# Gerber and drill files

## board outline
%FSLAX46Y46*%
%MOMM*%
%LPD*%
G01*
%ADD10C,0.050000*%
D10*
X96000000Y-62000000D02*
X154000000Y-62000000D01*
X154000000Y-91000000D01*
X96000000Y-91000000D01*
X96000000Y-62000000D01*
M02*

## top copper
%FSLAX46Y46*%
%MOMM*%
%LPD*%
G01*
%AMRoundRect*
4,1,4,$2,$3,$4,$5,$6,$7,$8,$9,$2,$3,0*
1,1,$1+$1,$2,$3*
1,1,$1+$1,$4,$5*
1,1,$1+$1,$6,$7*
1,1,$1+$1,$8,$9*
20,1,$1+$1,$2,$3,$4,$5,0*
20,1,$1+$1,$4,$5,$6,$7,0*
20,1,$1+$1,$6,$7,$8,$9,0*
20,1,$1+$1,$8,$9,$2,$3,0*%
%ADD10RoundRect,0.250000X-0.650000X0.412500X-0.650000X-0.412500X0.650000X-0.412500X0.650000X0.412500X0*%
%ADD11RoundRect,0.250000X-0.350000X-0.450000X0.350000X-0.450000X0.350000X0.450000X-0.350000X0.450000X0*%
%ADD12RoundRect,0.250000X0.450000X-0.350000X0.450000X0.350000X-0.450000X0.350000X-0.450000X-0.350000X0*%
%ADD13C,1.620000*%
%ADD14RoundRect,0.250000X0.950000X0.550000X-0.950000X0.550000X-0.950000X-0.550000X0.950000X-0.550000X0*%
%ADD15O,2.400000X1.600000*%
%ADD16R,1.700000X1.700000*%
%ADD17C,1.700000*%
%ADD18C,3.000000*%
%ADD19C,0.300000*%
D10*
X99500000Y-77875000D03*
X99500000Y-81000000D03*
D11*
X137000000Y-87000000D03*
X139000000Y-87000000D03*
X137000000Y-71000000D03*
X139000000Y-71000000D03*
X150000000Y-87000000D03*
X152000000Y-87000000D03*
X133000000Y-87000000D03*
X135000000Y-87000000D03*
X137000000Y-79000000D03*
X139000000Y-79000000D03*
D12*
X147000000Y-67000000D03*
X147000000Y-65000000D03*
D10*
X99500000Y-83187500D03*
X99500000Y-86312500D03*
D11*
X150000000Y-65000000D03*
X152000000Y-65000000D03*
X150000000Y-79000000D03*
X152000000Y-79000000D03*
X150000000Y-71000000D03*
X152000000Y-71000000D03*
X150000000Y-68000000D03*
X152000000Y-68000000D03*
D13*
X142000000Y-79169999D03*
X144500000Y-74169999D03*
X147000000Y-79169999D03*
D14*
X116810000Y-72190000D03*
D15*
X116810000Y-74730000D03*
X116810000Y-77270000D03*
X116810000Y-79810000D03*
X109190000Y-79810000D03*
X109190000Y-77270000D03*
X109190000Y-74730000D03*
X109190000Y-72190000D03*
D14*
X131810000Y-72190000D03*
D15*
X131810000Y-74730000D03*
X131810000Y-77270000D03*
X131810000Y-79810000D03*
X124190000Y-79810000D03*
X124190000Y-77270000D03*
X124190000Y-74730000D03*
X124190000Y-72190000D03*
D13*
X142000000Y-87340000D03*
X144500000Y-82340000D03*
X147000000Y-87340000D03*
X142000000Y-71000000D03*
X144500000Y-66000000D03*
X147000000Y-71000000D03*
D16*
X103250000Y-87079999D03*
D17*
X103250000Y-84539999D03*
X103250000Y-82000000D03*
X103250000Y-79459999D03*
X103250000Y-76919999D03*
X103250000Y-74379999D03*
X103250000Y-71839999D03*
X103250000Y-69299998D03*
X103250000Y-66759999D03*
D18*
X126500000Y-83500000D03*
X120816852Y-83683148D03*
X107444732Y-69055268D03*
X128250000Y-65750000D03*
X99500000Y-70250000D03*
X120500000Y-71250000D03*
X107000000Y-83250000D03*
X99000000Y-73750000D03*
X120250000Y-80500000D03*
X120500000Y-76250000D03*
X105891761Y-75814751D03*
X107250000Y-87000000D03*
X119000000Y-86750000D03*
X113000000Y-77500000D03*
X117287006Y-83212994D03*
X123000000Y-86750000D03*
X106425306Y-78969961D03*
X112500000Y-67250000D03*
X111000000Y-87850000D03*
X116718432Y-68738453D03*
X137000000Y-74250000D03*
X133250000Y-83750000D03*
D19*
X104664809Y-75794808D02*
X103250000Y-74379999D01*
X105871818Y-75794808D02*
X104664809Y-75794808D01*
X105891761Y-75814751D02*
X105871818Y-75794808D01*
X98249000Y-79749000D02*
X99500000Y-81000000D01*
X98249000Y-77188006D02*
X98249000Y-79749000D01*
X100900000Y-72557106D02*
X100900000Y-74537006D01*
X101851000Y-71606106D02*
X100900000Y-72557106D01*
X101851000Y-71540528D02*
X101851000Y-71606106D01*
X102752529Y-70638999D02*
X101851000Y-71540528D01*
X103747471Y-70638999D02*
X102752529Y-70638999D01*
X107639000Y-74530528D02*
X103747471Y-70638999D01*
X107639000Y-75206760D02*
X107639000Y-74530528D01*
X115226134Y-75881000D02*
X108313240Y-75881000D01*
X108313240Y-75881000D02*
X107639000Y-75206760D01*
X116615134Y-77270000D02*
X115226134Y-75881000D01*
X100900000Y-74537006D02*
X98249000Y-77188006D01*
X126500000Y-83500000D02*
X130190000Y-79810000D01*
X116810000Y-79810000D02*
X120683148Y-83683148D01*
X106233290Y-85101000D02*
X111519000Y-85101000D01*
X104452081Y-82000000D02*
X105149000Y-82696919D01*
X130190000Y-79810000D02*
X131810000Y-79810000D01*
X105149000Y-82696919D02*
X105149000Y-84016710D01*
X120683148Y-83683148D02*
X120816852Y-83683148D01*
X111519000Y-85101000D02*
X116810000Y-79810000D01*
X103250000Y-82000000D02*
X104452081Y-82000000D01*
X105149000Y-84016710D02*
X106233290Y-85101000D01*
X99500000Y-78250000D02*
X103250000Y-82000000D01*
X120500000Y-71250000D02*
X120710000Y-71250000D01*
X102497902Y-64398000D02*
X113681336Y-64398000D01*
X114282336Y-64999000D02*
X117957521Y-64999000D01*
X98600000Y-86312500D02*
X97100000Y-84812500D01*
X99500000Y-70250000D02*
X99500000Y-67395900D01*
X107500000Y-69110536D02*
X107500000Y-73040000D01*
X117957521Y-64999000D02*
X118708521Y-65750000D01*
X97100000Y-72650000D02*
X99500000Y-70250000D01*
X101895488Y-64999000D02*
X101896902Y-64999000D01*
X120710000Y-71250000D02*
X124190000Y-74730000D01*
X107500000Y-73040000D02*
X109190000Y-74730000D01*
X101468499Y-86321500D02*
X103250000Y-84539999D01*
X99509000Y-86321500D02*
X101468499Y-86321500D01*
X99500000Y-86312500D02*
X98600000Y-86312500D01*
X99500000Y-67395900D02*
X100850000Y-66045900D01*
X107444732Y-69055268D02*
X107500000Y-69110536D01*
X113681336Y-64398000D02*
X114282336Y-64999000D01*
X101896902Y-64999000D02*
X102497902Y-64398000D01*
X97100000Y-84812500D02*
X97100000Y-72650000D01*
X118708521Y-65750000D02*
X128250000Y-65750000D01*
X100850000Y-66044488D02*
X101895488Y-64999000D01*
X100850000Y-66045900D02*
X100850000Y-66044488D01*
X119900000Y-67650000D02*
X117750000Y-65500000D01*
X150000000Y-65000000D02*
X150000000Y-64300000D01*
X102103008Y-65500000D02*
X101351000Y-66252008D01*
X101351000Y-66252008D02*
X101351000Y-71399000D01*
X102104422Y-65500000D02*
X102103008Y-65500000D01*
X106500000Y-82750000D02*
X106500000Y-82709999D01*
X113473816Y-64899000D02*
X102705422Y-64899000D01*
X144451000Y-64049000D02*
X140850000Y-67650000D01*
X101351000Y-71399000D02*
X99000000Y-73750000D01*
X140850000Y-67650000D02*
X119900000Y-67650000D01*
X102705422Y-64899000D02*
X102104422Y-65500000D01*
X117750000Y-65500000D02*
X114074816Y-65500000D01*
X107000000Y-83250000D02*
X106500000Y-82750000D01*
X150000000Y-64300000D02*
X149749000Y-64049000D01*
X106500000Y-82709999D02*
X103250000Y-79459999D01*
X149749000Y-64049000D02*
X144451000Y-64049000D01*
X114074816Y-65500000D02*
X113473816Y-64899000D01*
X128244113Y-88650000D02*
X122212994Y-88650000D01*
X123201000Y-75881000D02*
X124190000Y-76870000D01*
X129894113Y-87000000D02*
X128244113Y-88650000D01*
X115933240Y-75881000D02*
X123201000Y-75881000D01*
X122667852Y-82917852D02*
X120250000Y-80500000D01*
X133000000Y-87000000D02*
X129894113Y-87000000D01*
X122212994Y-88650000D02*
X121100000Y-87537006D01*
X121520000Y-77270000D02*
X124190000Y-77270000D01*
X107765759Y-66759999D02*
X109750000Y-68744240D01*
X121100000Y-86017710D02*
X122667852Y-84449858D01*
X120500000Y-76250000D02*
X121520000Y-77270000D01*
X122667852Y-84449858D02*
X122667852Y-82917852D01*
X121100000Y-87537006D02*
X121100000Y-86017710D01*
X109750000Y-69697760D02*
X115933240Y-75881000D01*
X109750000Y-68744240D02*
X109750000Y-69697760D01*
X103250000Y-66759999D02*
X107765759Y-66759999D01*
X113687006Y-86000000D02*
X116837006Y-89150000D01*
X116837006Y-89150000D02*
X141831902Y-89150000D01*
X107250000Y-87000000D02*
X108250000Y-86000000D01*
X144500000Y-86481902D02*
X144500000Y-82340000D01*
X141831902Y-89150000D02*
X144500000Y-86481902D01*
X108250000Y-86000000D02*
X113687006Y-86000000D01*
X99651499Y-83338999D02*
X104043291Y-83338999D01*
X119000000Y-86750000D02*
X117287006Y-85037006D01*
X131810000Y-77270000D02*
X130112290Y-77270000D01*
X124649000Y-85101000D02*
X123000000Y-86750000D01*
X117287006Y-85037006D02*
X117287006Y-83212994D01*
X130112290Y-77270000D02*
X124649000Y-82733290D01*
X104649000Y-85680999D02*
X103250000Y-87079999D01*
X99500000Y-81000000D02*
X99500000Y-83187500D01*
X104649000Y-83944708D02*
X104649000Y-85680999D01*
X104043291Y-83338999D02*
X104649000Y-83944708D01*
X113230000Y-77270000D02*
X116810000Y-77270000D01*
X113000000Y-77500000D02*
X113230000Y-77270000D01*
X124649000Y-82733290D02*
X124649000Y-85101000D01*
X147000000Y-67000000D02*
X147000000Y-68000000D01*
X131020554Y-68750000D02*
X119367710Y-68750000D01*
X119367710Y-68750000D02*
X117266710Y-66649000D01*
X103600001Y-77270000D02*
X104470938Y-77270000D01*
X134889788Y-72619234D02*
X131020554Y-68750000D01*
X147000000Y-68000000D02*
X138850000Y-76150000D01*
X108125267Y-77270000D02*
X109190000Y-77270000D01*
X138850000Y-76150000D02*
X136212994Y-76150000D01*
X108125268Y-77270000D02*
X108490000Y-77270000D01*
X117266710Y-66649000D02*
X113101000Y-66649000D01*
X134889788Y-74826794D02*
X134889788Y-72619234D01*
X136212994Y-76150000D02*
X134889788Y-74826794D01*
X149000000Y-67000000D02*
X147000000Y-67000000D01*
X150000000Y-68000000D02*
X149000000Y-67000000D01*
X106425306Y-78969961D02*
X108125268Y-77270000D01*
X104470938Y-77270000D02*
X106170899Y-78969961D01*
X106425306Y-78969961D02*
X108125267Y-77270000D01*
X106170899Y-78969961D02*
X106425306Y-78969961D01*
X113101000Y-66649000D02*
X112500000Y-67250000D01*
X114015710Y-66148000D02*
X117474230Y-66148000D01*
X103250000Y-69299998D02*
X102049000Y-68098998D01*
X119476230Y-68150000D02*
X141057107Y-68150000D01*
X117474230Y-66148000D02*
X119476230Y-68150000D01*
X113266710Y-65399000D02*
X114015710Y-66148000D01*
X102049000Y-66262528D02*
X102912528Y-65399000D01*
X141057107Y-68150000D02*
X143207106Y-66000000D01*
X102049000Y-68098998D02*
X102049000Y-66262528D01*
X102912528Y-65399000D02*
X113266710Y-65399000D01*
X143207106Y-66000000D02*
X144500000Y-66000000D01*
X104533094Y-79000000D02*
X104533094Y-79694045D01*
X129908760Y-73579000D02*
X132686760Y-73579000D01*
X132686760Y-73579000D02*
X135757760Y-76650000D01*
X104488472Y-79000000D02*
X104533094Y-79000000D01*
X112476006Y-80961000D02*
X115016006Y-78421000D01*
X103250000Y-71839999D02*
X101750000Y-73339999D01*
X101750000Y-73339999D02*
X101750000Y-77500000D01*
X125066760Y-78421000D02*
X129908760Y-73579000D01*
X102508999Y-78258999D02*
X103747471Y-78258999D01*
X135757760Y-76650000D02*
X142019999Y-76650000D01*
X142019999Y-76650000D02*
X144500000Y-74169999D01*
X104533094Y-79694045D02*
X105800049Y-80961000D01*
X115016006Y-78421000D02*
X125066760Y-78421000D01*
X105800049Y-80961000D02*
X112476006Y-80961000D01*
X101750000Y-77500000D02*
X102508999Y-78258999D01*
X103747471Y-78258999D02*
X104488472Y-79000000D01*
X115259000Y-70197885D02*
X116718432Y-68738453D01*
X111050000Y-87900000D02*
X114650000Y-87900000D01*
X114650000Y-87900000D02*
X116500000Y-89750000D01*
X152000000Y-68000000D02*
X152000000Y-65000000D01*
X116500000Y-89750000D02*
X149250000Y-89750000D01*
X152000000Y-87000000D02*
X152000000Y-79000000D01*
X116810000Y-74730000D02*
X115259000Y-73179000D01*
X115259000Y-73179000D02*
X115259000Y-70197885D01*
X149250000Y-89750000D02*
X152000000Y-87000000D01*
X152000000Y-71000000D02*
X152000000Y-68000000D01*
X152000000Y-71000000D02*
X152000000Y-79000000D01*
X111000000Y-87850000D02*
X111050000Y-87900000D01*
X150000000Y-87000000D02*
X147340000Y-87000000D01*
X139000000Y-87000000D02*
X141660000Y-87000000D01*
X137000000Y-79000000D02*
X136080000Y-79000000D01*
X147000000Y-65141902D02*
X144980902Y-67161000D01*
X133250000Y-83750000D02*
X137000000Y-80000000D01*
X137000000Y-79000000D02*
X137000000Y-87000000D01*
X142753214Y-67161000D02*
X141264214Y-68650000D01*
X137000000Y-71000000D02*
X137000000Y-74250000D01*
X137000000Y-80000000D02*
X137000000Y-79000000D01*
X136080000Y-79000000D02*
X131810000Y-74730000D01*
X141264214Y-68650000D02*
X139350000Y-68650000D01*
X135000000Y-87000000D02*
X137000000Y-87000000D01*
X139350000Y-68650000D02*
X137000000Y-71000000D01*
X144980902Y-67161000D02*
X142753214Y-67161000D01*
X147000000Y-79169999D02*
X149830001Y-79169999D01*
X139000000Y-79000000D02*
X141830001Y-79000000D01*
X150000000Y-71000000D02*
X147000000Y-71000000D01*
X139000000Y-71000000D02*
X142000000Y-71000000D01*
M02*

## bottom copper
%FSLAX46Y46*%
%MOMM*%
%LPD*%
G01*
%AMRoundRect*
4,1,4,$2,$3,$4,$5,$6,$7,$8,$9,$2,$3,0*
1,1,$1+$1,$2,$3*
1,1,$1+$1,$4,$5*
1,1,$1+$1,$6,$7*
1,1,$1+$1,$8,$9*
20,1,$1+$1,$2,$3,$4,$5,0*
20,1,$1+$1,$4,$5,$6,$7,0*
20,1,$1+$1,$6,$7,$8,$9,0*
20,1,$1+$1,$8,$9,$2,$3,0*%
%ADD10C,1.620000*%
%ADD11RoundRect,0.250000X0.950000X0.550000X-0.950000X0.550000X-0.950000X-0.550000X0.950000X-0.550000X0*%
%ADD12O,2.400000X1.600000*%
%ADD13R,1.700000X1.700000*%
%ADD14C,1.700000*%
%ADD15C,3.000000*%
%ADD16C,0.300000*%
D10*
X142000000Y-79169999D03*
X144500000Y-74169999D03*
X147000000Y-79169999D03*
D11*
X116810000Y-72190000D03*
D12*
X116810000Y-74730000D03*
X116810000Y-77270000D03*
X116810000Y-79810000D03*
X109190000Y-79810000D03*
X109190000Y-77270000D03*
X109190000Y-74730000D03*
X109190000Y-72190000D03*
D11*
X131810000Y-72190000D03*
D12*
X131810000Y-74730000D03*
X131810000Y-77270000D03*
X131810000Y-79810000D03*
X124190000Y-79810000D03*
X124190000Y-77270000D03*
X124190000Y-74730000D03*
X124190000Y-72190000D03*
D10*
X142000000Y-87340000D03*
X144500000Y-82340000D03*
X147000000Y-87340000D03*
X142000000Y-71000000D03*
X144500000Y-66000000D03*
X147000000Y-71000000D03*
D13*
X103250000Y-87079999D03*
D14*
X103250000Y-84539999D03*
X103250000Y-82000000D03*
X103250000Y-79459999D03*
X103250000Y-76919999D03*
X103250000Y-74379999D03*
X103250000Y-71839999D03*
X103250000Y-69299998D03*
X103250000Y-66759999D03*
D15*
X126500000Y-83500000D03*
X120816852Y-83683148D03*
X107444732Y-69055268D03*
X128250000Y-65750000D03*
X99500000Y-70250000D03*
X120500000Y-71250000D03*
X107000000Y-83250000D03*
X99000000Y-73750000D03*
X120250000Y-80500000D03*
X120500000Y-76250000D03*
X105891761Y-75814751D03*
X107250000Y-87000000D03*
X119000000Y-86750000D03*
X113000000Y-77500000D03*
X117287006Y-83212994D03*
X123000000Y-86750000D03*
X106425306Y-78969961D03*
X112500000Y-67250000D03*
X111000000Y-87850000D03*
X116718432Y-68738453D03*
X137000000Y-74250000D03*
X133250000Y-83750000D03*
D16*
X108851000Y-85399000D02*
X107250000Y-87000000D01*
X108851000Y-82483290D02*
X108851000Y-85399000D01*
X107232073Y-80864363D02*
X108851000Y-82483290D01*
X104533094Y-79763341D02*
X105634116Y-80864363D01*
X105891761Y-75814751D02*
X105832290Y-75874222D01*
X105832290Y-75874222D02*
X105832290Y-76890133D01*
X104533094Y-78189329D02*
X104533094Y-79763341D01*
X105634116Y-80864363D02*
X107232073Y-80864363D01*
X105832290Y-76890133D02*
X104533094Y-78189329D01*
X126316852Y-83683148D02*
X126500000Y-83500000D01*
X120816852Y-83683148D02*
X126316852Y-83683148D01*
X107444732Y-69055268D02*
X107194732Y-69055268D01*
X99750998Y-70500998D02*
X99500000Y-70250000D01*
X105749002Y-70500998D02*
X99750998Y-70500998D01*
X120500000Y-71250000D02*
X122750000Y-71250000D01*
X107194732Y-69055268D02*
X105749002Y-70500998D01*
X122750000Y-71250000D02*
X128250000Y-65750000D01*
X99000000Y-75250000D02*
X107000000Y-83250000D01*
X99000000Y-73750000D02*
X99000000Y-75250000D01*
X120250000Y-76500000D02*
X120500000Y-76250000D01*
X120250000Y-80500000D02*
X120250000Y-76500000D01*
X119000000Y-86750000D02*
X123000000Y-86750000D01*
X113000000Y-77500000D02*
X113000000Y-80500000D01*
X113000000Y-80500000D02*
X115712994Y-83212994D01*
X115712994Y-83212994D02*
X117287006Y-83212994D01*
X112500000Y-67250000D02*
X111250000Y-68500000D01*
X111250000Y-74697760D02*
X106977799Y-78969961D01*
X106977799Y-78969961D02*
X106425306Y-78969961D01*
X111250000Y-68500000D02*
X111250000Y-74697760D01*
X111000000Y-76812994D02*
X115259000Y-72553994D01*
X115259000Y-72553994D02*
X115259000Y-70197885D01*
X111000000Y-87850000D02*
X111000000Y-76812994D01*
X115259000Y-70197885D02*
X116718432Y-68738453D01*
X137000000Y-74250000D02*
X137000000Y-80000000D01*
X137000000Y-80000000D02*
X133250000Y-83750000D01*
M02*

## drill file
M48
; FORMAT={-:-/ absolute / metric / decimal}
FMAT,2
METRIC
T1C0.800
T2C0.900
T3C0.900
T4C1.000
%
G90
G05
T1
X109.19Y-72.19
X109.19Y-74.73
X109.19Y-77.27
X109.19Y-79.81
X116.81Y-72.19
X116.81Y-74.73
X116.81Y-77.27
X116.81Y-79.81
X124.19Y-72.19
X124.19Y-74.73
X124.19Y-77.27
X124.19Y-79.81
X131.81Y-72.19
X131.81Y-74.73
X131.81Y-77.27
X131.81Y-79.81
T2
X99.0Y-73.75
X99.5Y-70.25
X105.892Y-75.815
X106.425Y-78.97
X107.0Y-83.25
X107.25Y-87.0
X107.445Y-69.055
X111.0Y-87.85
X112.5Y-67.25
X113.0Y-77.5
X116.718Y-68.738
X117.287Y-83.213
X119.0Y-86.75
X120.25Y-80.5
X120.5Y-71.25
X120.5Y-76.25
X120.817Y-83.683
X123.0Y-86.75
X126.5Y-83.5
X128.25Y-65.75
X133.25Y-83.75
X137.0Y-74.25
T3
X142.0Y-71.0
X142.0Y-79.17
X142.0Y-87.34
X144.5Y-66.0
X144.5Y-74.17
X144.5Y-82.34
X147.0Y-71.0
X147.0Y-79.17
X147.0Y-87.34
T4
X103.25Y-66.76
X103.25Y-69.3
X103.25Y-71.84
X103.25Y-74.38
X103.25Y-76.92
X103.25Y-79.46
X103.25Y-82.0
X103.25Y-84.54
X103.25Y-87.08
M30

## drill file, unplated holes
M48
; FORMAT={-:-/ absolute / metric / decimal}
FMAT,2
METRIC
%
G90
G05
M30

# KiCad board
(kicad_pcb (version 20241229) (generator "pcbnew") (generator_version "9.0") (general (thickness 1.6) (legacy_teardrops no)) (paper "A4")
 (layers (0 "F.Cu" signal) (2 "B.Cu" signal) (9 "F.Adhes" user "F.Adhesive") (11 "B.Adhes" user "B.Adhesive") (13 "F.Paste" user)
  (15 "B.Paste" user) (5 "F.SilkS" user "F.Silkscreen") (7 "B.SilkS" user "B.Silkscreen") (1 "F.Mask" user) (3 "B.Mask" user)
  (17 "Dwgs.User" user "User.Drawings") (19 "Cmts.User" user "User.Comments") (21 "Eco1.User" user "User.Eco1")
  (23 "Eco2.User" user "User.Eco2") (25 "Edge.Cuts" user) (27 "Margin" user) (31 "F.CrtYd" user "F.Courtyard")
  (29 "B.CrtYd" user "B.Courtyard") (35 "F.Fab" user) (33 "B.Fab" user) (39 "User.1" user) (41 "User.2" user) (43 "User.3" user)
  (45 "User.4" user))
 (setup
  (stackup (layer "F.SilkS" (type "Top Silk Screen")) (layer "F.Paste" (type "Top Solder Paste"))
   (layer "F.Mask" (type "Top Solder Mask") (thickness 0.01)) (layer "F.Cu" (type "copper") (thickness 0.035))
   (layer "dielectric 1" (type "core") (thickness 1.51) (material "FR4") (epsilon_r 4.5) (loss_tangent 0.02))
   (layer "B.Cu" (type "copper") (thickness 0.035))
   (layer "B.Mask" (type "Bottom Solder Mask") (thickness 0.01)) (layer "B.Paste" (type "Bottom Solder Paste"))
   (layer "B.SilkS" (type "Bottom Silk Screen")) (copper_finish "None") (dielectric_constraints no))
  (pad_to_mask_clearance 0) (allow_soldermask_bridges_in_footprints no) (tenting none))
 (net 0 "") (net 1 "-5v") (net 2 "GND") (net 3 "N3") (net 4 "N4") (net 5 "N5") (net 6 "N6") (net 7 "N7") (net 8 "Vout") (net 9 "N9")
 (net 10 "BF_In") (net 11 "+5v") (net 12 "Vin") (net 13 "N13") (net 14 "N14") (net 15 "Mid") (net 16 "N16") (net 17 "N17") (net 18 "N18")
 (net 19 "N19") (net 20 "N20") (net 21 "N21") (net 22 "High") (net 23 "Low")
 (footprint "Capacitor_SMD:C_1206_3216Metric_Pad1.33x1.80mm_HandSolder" (layer "F.Cu") (at 99.5 79.4375 -90)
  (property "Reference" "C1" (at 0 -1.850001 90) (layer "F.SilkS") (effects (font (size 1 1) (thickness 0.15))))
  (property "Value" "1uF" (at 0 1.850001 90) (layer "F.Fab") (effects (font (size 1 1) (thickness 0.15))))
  (pad "1" smd roundrect (at -1.5625 0 270) (size 1.325 1.8) (layers "F.Cu" "F.Mask" "F.Paste") (roundrect_rratio 0.188679) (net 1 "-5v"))
  (pad "2" smd roundrect (at 1.5625 0 270) (size 1.325 1.8) (layers "F.Cu" "F.Mask" "F.Paste") (roundrect_rratio 0.188679) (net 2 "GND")))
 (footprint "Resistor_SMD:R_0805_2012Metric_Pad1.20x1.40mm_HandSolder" (layer "F.Cu") (at 138 87)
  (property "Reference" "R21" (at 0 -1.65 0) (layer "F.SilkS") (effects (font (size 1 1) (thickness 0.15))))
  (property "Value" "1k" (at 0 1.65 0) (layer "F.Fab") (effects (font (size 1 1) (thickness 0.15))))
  (pad "1" smd roundrect (at -1 0) (size 1.2 1.4) (layers "F.Cu" "F.Mask" "F.Paste") (roundrect_rratio 0.208333) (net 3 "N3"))
  (pad "2" smd roundrect (at 1 0) (size 1.2 1.4) (layers "F.Cu" "F.Mask" "F.Paste") (roundrect_rratio 0.208333) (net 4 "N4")))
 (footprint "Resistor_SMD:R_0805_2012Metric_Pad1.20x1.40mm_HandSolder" (layer "F.Cu") (at 138 71)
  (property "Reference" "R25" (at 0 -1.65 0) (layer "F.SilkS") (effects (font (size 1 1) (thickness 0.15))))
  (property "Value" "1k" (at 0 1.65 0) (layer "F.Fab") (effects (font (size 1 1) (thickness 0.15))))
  (pad "1" smd roundrect (at -1 0) (size 1.2 1.4) (layers "F.Cu" "F.Mask" "F.Paste") (roundrect_rratio 0.208333) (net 3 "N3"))
  (pad "2" smd roundrect (at 1 0) (size 1.2 1.4) (layers "F.Cu" "F.Mask" "F.Paste") (roundrect_rratio 0.208333) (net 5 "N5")))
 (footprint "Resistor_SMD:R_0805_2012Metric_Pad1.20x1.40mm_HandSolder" (layer "F.Cu") (at 151 87)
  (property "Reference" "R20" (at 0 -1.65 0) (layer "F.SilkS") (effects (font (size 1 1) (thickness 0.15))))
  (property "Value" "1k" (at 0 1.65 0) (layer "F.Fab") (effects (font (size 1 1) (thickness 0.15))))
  (pad "1" smd roundrect (at -1 0) (size 1.2 1.4) (layers "F.Cu" "F.Mask" "F.Paste") (roundrect_rratio 0.208333) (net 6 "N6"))
  (pad "2" smd roundrect (at 1 0) (size 1.2 1.4) (layers "F.Cu" "F.Mask" "F.Paste") (roundrect_rratio 0.208333) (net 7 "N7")))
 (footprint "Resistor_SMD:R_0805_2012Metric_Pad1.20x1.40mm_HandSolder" (layer "F.Cu") (at 134 87)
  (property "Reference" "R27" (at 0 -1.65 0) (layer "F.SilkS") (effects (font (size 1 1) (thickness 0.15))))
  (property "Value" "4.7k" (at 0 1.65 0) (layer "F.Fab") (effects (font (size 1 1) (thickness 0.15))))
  (pad "1" smd roundrect (at -1 0) (size 1.2 1.4) (layers "F.Cu" "F.Mask" "F.Paste") (roundrect_rratio 0.208333) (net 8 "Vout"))
  (pad "2" smd roundrect (at 1 0) (size 1.2 1.4) (layers "F.Cu" "F.Mask" "F.Paste") (roundrect_rratio 0.208333) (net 3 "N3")))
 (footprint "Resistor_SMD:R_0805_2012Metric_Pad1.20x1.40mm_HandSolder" (layer "F.Cu") (at 138 79)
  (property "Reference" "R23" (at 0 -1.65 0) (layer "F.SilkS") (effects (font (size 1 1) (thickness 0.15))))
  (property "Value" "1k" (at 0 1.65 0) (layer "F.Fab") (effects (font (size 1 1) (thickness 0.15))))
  (pad "1" smd roundrect (at -1 0) (size 1.2 1.4) (layers "F.Cu" "F.Mask" "F.Paste") (roundrect_rratio 0.208333) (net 3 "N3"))
  (pad "2" smd roundrect (at 1 0) (size 1.2 1.4) (layers "F.Cu" "F.Mask" "F.Paste") (roundrect_rratio 0.208333) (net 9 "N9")))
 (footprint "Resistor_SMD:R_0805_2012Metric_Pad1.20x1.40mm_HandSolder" (layer "F.Cu") (at 147 66 90)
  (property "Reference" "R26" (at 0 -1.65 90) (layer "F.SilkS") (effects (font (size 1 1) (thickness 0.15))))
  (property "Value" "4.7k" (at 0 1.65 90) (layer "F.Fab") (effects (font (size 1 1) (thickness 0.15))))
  (pad "1" smd roundrect (at -1 0 90) (size 1.2 1.4) (layers "F.Cu" "F.Mask" "F.Paste") (roundrect_rratio 0.208333) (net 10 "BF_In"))
  (pad "2" smd roundrect (at 1 0 90) (size 1.2 1.4) (layers "F.Cu" "F.Mask" "F.Paste") (roundrect_rratio 0.208333) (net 3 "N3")))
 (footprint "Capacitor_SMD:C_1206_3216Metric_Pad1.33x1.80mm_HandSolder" (layer "F.Cu") (at 99.5 84.75 -90)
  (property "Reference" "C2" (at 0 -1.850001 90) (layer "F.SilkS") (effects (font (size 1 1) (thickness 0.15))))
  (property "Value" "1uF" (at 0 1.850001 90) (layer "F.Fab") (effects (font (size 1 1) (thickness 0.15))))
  (pad "1" smd roundrect (at -1.5625 0 270) (size 1.325 1.8) (layers "F.Cu" "F.Mask" "F.Paste") (roundrect_rratio 0.188679) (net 2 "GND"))
  (pad "2" smd roundrect (at 1.5625 0 270) (size 1.325 1.8) (layers "F.Cu" "F.Mask" "F.Paste") (roundrect_rratio 0.188679) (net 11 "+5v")))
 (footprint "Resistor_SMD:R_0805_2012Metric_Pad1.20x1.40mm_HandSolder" (layer "F.Cu") (at 151 65)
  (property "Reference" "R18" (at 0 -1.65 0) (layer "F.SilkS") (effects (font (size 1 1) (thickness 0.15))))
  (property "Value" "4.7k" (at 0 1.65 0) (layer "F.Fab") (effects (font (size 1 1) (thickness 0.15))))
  (pad "1" smd roundrect (at -1 0) (size 1.2 1.4) (layers "F.Cu" "F.Mask" "F.Paste") (roundrect_rratio 0.208333) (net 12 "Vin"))
  (pad "2" smd roundrect (at 1 0) (size 1.2 1.4) (layers "F.Cu" "F.Mask" "F.Paste") (roundrect_rratio 0.208333) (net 7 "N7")))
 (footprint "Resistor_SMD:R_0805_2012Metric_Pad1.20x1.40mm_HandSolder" (layer "F.Cu") (at 151 79)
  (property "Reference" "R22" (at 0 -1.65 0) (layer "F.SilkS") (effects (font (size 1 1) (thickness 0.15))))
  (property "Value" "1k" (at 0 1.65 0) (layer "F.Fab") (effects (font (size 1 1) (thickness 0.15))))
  (pad "1" smd roundrect (at -1 0) (size 1.2 1.4) (layers "F.Cu" "F.Mask" "F.Paste") (roundrect_rratio 0.208333) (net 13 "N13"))
  (pad "2" smd roundrect (at 1 0) (size 1.2 1.4) (layers "F.Cu" "F.Mask" "F.Paste") (roundrect_rratio 0.208333) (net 7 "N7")))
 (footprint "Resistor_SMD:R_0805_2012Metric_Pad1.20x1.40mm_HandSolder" (layer "F.Cu") (at 151 71)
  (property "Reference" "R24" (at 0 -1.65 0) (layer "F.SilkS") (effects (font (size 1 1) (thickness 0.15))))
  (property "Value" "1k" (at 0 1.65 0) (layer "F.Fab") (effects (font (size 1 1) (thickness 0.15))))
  (pad "1" smd roundrect (at -1 0) (size 1.2 1.4) (layers "F.Cu" "F.Mask" "F.Paste") (roundrect_rratio 0.208333) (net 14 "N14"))
  (pad "2" smd roundrect (at 1 0) (size 1.2 1.4) (layers "F.Cu" "F.Mask" "F.Paste") (roundrect_rratio 0.208333) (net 7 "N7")))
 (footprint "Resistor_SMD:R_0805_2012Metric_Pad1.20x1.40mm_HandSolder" (layer "F.Cu") (at 151 68)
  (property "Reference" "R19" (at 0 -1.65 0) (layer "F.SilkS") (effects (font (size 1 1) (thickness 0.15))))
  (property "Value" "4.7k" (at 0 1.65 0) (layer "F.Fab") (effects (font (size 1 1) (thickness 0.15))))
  (pad "1" smd roundrect (at -1 0) (size 1.2 1.4) (layers "F.Cu" "F.Mask" "F.Paste") (roundrect_rratio 0.208333) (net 10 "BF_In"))
  (pad "2" smd roundrect (at 1 0) (size 1.2 1.4) (layers "F.Cu" "F.Mask" "F.Paste") (roundrect_rratio 0.208333) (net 7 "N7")))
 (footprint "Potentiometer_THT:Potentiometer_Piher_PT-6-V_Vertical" (layer "B.Cu") (at 142 79.169999 90)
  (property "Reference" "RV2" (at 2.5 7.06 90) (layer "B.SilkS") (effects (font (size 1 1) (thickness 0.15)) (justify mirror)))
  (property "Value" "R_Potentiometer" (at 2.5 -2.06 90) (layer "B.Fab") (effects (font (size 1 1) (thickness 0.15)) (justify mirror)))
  (pad "1" thru_hole circle (at 0 0 90) (size 1.62 1.62) (drill 0.9) (layers "*.Cu" "*.Mask") (remove_unused_layers no) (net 9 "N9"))
  (pad "2" thru_hole circle (at 5 2.5 90) (size 1.62 1.62) (drill 0.9) (layers "*.Cu" "*.Mask") (remove_unused_layers no) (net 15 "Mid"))
  (pad "3" thru_hole circle (at 0 5 90) (size 1.62 1.62) (drill 0.9) (layers "*.Cu" "*.Mask") (remove_unused_layers no) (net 13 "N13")))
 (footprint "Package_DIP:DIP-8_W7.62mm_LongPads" (layer "B.Cu") (at 116.81 72.19 180)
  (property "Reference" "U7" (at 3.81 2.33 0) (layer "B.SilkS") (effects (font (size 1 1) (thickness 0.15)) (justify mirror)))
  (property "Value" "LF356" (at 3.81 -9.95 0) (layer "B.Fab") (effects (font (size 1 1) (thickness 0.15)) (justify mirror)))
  (pad "1" thru_hole roundrect (at 0 0 180) (size 2.4 1.6) (drill 0.8) (layers "*.Cu" "*.Mask") (remove_unused_layers no)
   (roundrect_rratio 0.15625) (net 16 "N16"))
  (pad "2" thru_hole oval (at 0 -2.54 180) (size 2.4 1.6) (drill 0.8) (layers "*.Cu" "*.Mask") (remove_unused_layers no) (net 7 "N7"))
  (pad "3" thru_hole oval (at 0 -5.08 180) (size 2.4 1.6) (drill 0.8) (layers "*.Cu" "*.Mask") (remove_unused_layers no) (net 2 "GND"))
  (pad "4" thru_hole oval (at 0 -7.62 180) (size 2.4 1.6) (drill 0.8) (layers "*.Cu" "*.Mask") (remove_unused_layers no) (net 1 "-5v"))
  (pad "5" thru_hole oval (at 7.62 -7.62 180) (size 2.4 1.6) (drill 0.8) (layers "*.Cu" "*.Mask") (remove_unused_layers no) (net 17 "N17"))
  (pad "6" thru_hole oval (at 7.62 -5.08 180) (size 2.4 1.6) (drill 0.8) (layers "*.Cu" "*.Mask") (remove_unused_layers no) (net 10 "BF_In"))
  (pad "7" thru_hole oval (at 7.62 -2.54 180) (size 2.4 1.6) (drill 0.8) (layers "*.Cu" "*.Mask") (remove_unused_layers no) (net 11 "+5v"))
  (pad "8" thru_hole oval (at 7.62 0 180) (size 2.4 1.6) (drill 0.8) (layers "*.Cu" "*.Mask") (remove_unused_layers no) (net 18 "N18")))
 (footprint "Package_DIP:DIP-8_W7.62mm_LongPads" (layer "B.Cu") (at 131.81 72.19 180)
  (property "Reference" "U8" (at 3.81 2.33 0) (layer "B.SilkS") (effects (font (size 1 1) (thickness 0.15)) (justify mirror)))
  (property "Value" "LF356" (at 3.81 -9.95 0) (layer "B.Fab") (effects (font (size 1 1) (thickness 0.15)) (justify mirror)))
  (pad "1" thru_hole roundrect (at 0 0 180) (size 2.4 1.6) (drill 0.8) (layers "*.Cu" "*.Mask") (remove_unused_layers no)
   (roundrect_rratio 0.15625) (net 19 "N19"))
  (pad "2" thru_hole oval (at 0 -2.54 180) (size 2.4 1.6) (drill 0.8) (layers "*.Cu" "*.Mask") (remove_unused_layers no) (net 3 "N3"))
  (pad "3" thru_hole oval (at 0 -5.08 180) (size 2.4 1.6) (drill 0.8) (layers "*.Cu" "*.Mask") (remove_unused_layers no) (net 2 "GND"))
  (pad "4" thru_hole oval (at 0 -7.62 180) (size 2.4 1.6) (drill 0.8) (layers "*.Cu" "*.Mask") (remove_unused_layers no) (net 1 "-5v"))
  (pad "5" thru_hole oval (at 7.62 -7.62 180) (size 2.4 1.6) (drill 0.8) (layers "*.Cu" "*.Mask") (remove_unused_layers no) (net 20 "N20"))
  (pad "6" thru_hole oval (at 7.62 -5.08 180) (size 2.4 1.6) (drill 0.8) (layers "*.Cu" "*.Mask") (remove_unused_layers no) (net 8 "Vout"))
  (pad "7" thru_hole oval (at 7.62 -2.54 180) (size 2.4 1.6) (drill 0.8) (layers "*.Cu" "*.Mask") (remove_unused_layers no) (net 11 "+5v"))
  (pad "8" thru_hole oval (at 7.62 0 180) (size 2.4 1.6) (drill 0.8) (layers "*.Cu" "*.Mask") (remove_unused_layers no) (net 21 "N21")))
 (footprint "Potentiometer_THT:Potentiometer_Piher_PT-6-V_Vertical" (layer "B.Cu") (at 142 87.34 90)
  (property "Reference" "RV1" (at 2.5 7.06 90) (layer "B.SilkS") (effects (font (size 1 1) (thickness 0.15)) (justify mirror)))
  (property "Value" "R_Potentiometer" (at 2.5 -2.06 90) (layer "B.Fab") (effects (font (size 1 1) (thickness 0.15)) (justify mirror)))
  (pad "1" thru_hole circle (at 0 0 90) (size 1.62 1.62) (drill 0.9) (layers "*.Cu" "*.Mask") (remove_unused_layers no) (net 4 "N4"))
  (pad "2" thru_hole circle (at 5 2.5 90) (size 1.62 1.62) (drill 0.9) (layers "*.Cu" "*.Mask") (remove_unused_layers no) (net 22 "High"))
  (pad "3" thru_hole circle (at 0 5 90) (size 1.62 1.62) (drill 0.9) (layers "*.Cu" "*.Mask") (remove_unused_layers no) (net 6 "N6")))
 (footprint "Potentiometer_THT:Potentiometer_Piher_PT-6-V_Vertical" (layer "B.Cu") (at 142 71 90)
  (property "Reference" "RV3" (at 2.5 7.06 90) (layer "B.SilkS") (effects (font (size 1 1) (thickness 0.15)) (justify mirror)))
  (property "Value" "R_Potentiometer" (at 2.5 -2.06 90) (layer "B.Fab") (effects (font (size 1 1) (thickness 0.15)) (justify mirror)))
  (pad "1" thru_hole circle (at 0 0 90) (size 1.62 1.62) (drill 0.9) (layers "*.Cu" "*.Mask") (remove_unused_layers no) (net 5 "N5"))
  (pad "2" thru_hole circle (at 5 2.5 90) (size 1.62 1.62) (drill 0.9) (layers "*.Cu" "*.Mask") (remove_unused_layers no) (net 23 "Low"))
  (pad "3" thru_hole circle (at 0 5 90) (size 1.62 1.62) (drill 0.9) (layers "*.Cu" "*.Mask") (remove_unused_layers no) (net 14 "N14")))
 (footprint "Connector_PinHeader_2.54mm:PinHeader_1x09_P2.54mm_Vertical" (layer "B.Cu") (at 103.25 87.079999)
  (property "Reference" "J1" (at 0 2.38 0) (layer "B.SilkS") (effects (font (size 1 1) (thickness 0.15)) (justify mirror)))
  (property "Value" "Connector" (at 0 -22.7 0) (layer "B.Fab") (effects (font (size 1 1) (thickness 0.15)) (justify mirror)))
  (pad "1" thru_hole rect (at 0 0) (size 1.7 1.7) (drill 1) (layers "*.Cu" "*.Mask") (remove_unused_layers no) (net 2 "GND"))
  (pad "2" thru_hole circle (at 0 -2.54) (size 1.7 1.7) (drill 1) (layers "*.Cu" "*.Mask") (remove_unused_layers no) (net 11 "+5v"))
  (pad "3" thru_hole circle (at 0 -5.079999) (size 1.7 1.7) (drill 1) (layers "*.Cu" "*.Mask") (remove_unused_layers no) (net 1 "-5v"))
  (pad "4" thru_hole circle (at 0 -7.62) (size 1.7 1.7) (drill 1) (layers "*.Cu" "*.Mask") (remove_unused_layers no) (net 12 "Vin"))
  (pad "5" thru_hole circle (at 0 -10.16) (size 1.7 1.7) (drill 1) (layers "*.Cu" "*.Mask") (remove_unused_layers no) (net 10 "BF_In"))
  (pad "6" thru_hole circle (at 0 -12.7) (size 1.7 1.7) (drill 1) (layers "*.Cu" "*.Mask") (remove_unused_layers no) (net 22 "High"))
  (pad "7" thru_hole circle (at 0 -15.24) (size 1.7 1.7) (drill 1) (layers "*.Cu" "*.Mask") (remove_unused_layers no) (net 15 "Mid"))
  (pad "8" thru_hole circle (at 0 -17.780001) (size 1.7 1.7) (drill 1) (layers "*.Cu" "*.Mask") (remove_unused_layers no) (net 23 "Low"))
  (pad "9" thru_hole circle (at 0 -20.32) (size 1.7 1.7) (drill 1) (layers "*.Cu" "*.Mask") (remove_unused_layers no) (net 8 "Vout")))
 (gr_rect (start 96 62) (end 154 91) (stroke (width 0.05) (type default)) (fill no) (layer "Edge.Cuts"))
 (segment (start 126.5 83.5) (end 130.19 79.81) (width 0.3) (layer "F.Cu") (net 1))
 (segment (start 116.81 79.81) (end 120.683148 83.683148) (width 0.3) (layer "F.Cu") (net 1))
 (segment (start 106.23329 85.101) (end 111.519 85.101) (width 0.3) (layer "F.Cu") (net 1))
 (segment (start 104.452081 82) (end 105.149 82.696919) (width 0.3) (layer "F.Cu") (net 1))
 (segment (start 130.19 79.81) (end 131.81 79.81) (width 0.3) (layer "F.Cu") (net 1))
 (segment (start 105.149 82.696919) (end 105.149 84.01671) (width 0.3) (layer "F.Cu") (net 1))
 (segment (start 120.683148 83.683148) (end 120.816852 83.683148) (width 0.3) (layer "F.Cu") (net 1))
 (segment (start 111.519 85.101) (end 116.81 79.81) (width 0.3) (layer "F.Cu") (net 1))
 (segment (start 103.25 82) (end 104.452081 82) (width 0.3) (layer "F.Cu") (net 1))
 (segment (start 105.149 84.01671) (end 106.23329 85.101) (width 0.3) (layer "F.Cu") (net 1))
 (segment (start 99.5 78.25) (end 103.25 82) (width 0.3) (layer "F.Cu") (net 1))
 (via (at 126.5 83.5) (size 3) (drill 0.9) (layers "F.Cu" "B.Cu") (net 1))
 (via (at 120.816852 83.683148) (size 3) (drill 0.9) (layers "F.Cu" "B.Cu") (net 1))
 (segment (start 126.316852 83.683148) (end 126.5 83.5) (width 0.3) (layer "B.Cu") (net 1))
 (segment (start 120.816852 83.683148) (end 126.316852 83.683148) (width 0.3) (layer "B.Cu") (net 1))
 (segment (start 120.5 71.25) (end 120.71 71.25) (width 0.3) (layer "F.Cu") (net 11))
 (segment (start 102.497902 64.398) (end 113.681336 64.398) (width 0.3) (layer "F.Cu") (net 11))
 (segment (start 114.282336 64.999) (end 117.957521 64.999) (width 0.3) (layer "F.Cu") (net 11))
 (segment (start 98.6 86.3125) (end 97.1 84.8125) (width 0.3) (layer "F.Cu") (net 11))
 (segment (start 99.5 70.25) (end 99.5 67.3959) (width 0.3) (layer "F.Cu") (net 11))
 (segment (start 107.5 69.110536) (end 107.5 73.04) (width 0.3) (layer "F.Cu") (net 11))
 (segment (start 117.957521 64.999) (end 118.708521 65.75) (width 0.3) (layer "F.Cu") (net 11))
 (segment (start 97.1 72.65) (end 99.5 70.25) (width 0.3) (layer "F.Cu") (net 11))
 (segment (start 101.895488 64.999) (end 101.896902 64.999) (width 0.3) (layer "F.Cu") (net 11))
 (segment (start 120.71 71.25) (end 124.19 74.73) (width 0.3) (layer "F.Cu") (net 11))
 (segment (start 107.5 73.04) (end 109.19 74.73) (width 0.3) (layer "F.Cu") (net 11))
 (segment (start 101.468499 86.3215) (end 103.25 84.539999) (width 0.3) (layer "F.Cu") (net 11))
 (segment (start 99.509 86.3215) (end 101.468499 86.3215) (width 0.3) (layer "F.Cu") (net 11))
 (segment (start 99.5 86.3125) (end 98.6 86.3125) (width 0.3) (layer "F.Cu") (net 11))
 (segment (start 99.5 67.3959) (end 100.85 66.0459) (width 0.3) (layer "F.Cu") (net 11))
 (segment (start 107.444732 69.055268) (end 107.5 69.110536) (width 0.3) (layer "F.Cu") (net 11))
 (segment (start 113.681336 64.398) (end 114.282336 64.999) (width 0.3) (layer "F.Cu") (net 11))
 (segment (start 101.896902 64.999) (end 102.497902 64.398) (width 0.3) (layer "F.Cu") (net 11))
 (segment (start 97.1 84.8125) (end 97.1 72.65) (width 0.3) (layer "F.Cu") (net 11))
 (segment (start 118.708521 65.75) (end 128.25 65.75) (width 0.3) (layer "F.Cu") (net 11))
 (segment (start 100.85 66.044488) (end 101.895488 64.999) (width 0.3) (layer "F.Cu") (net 11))
 (segment (start 100.85 66.0459) (end 100.85 66.044488) (width 0.3) (layer "F.Cu") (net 11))
 (via (at 107.444732 69.055268) (size 3) (drill 0.9) (layers "F.Cu" "B.Cu") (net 11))
 (via (at 128.25 65.75) (size 3) (drill 0.9) (layers "F.Cu" "B.Cu") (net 11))
 (via (at 99.5 70.25) (size 3) (drill 0.9) (layers "F.Cu" "B.Cu") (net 11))
 (via (at 120.5 71.25) (size 3) (drill 0.9) (layers "F.Cu" "B.Cu") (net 11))
 (segment (start 107.444732 69.055268) (end 107.194732 69.055268) (width 0.3) (layer "B.Cu") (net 11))
 (segment (start 99.750998 70.500998) (end 99.5 70.25) (width 0.3) (layer "B.Cu") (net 11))
 (segment (start 105.749002 70.500998) (end 99.750998 70.500998) (width 0.3) (layer "B.Cu") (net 11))
 (segment (start 120.5 71.25) (end 122.75 71.25) (width 0.3) (layer "B.Cu") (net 11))
 (segment (start 107.194732 69.055268) (end 105.749002 70.500998) (width 0.3) (layer "B.Cu") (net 11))
 (segment (start 122.75 71.25) (end 128.25 65.75) (width 0.3) (layer "B.Cu") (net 11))
 (segment (start 119.9 67.65) (end 117.75 65.5) (width 0.3) (layer "F.Cu") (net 12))
 (segment (start 150 65) (end 150 64.3) (width 0.3) (layer "F.Cu") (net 12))
 (segment (start 102.103008 65.5) (end 101.351 66.252008) (width 0.3) (layer "F.Cu") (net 12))
 (segment (start 101.351 66.252008) (end 101.351 71.399) (width 0.3) (layer "F.Cu") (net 12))
 (segment (start 102.104422 65.5) (end 102.103008 65.5) (width 0.3) (layer "F.Cu") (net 12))
 (segment (start 106.5 82.75) (end 106.5 82.709999) (width 0.3) (layer "F.Cu") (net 12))
 (segment (start 113.473816 64.899) (end 102.705422 64.899) (width 0.3) (layer "F.Cu") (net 12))
 (segment (start 144.451 64.049) (end 140.85 67.65) (width 0.3) (layer "F.Cu") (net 12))
 (segment (start 101.351 71.399) (end 99 73.75) (width 0.3) (layer "F.Cu") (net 12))
 (segment (start 140.85 67.65) (end 119.9 67.65) (width 0.3) (layer "F.Cu") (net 12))
 (segment (start 102.705422 64.899) (end 102.104422 65.5) (width 0.3) (layer "F.Cu") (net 12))
 (segment (start 117.75 65.5) (end 114.074816 65.5) (width 0.3) (layer "F.Cu") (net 12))
 (segment (start 107 83.25) (end 106.5 82.75) (width 0.3) (layer "F.Cu") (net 12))
 (segment (start 150 64.3) (end 149.749 64.049) (width 0.3) (layer "F.Cu") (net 12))
 (segment (start 106.5 82.709999) (end 103.25 79.459999) (width 0.3) (layer "F.Cu") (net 12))
 (segment (start 149.749 64.049) (end 144.451 64.049) (width 0.3) (layer "F.Cu") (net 12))
 (segment (start 114.074816 65.5) (end 113.473816 64.899) (width 0.3) (layer "F.Cu") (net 12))
 (via (at 107 83.25) (size 3) (drill 0.9) (layers "F.Cu" "B.Cu") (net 12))
 (via (at 99 73.75) (size 3) (drill 0.9) (layers "F.Cu" "B.Cu") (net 12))
 (segment (start 99 76.75) (end 103.049 80.799) (width 0.3) (layer "B.Cu") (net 12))
 (segment (start 103.049 80.799) (end 103.747471 80.799) (width 0.3) (layer "B.Cu") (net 12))
 (segment (start 106.198471 83.25) (end 107 83.25) (width 0.3) (layer "B.Cu") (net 12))
 (segment (start 103.747471 80.799) (end 106.198471 83.25) (width 0.3) (layer "B.Cu") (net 12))
 (segment (start 99 73.75) (end 99 76.75) (width 0.3) (layer "B.Cu") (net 12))
 (segment (start 128.244113 88.65) (end 122.212994 88.65) (width 0.3) (layer "F.Cu") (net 8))
 (segment (start 123.201 75.881) (end 124.19 76.87) (width 0.3) (layer "F.Cu") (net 8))
 (segment (start 129.894113 87) (end 128.244113 88.65) (width 0.3) (layer "F.Cu") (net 8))
 (segment (start 115.93324 75.881) (end 123.201 75.881) (width 0.3) (layer "F.Cu") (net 8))
 (segment (start 122.667852 82.917852) (end 120.25 80.5) (width 0.3) (layer "F.Cu") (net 8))
 (segment (start 133 87) (end 129.894113 87) (width 0.3) (layer "F.Cu") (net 8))
 (segment (start 122.212994 88.65) (end 121.1 87.537006) (width 0.3) (layer "F.Cu") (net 8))
 (segment (start 121.52 77.27) (end 124.19 77.27) (width 0.3) (layer "F.Cu") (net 8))
 (segment (start 107.765759 66.759999) (end 109.75 68.74424) (width 0.3) (layer "F.Cu") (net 8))
 (segment (start 121.1 86.01771) (end 122.667852 84.449858) (width 0.3) (layer "F.Cu") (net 8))
 (segment (start 120.5 76.25) (end 121.52 77.27) (width 0.3) (layer "F.Cu") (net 8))
 (segment (start 122.667852 84.449858) (end 122.667852 82.917852) (width 0.3) (layer "F.Cu") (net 8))
 (segment (start 121.1 87.537006) (end 121.1 86.01771) (width 0.3) (layer "F.Cu") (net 8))
 (segment (start 109.75 69.69776) (end 115.93324 75.881) (width 0.3) (layer "F.Cu") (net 8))
 (segment (start 109.75 68.74424) (end 109.75 69.69776) (width 0.3) (layer "F.Cu") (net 8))
 (segment (start 103.25 66.759999) (end 107.765759 66.759999) (width 0.3) (layer "F.Cu") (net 8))
 (via (at 120.25 80.5) (size 3) (drill 0.9) (layers "F.Cu" "B.Cu") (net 8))
 (via (at 120.5 76.25) (size 3) (drill 0.9) (layers "F.Cu" "B.Cu") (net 8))
 (segment (start 120.25 76.5) (end 120.5 76.25) (width 0.3) (layer "B.Cu") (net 8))
 (segment (start 120.25 80.5) (end 120.25 76.5) (width 0.3) (layer "B.Cu") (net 8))
 (segment (start 113.687006 86) (end 116.837006 89.15) (width 0.3) (layer "F.Cu") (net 22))
 (segment (start 116.837006 89.15) (end 141.831902 89.15) (width 0.3) (layer "F.Cu") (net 22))
 (segment (start 107.25 87) (end 108.25 86) (width 0.3) (layer "F.Cu") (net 22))
 (segment (start 105.871818 75.794808) (end 104.664809 75.794808) (width 0.3) (layer "F.Cu") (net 22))
 (segment (start 144.5 86.481902) (end 144.5 82.34) (width 0.3) (layer "F.Cu") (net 22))
 (segment (start 105.891761 75.814751) (end 105.871818 75.794808) (width 0.3) (layer "F.Cu") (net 22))
 (segment (start 141.831902 89.15) (end 144.5 86.481902) (width 0.3) (layer "F.Cu") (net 22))
 (segment (start 108.25 86) (end 113.687006 86) (width 0.3) (layer "F.Cu") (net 22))
 (segment (start 104.664809 75.794808) (end 103.25 74.379999) (width 0.3) (layer "F.Cu") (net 22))
 (via (at 105.891761 75.814751) (size 3) (drill 0.9) (layers "F.Cu" "B.Cu") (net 22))
 (via (at 107.25 87) (size 3) (drill 0.9) (layers "F.Cu" "B.Cu") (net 22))
 (segment (start 105.83229 75.874222) (end 105.83229 76.890133) (width 0.3) (layer "B.Cu") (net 22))
 (segment (start 105.83229 76.890133) (end 104.533094 78.189329) (width 0.3) (layer "B.Cu") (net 22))
 (segment (start 104.533094 78.189329) (end 104.533094 79.763341) (width 0.3) (layer "B.Cu") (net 22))
 (segment (start 108.851 85.399) (end 107.25 87) (width 0.3) (layer "B.Cu") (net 22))
 (segment (start 105.891761 75.814751) (end 105.83229 75.874222) (width 0.3) (layer "B.Cu") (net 22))
 (segment (start 105.634116 80.864363) (end 107.232073 80.864363) (width 0.3) (layer "B.Cu") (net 22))
 (segment (start 107.232073 80.864363) (end 108.851 82.48329) (width 0.3) (layer "B.Cu") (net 22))
 (segment (start 104.533094 79.763341) (end 105.634116 80.864363) (width 0.3) (layer "B.Cu") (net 22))
 (segment (start 108.851 82.48329) (end 108.851 85.399) (width 0.3) (layer "B.Cu") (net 22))
 (segment (start 99.651499 83.338999) (end 104.043291 83.338999) (width 0.3) (layer "F.Cu") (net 2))
 (segment (start 119 86.75) (end 117.287006 85.037006) (width 0.3) (layer "F.Cu") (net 2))
 (segment (start 131.81 77.27) (end 130.11229 77.27) (width 0.3) (layer "F.Cu") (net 2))
 (segment (start 124.649 85.101) (end 123 86.75) (width 0.3) (layer "F.Cu") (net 2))
 (segment (start 102.752529 70.638999) (end 101.851 71.540528) (width 0.3) (layer "F.Cu") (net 2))
 (segment (start 117.287006 85.037006) (end 117.287006 83.212994) (width 0.3) (layer "F.Cu") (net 2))
 (segment (start 101.851 71.540528) (end 101.851 71.606106) (width 0.3) (layer "F.Cu") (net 2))
 (segment (start 103.747471 70.638999) (end 102.752529 70.638999) (width 0.3) (layer "F.Cu") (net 2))
 (segment (start 100.9 72.557106) (end 100.9 74.537006) (width 0.3) (layer "F.Cu") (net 2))
 (segment (start 130.11229 77.27) (end 124.649 82.73329) (width 0.3) (layer "F.Cu") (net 2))
 (segment (start 116.615134 77.27) (end 115.226134 75.881) (width 0.3) (layer "F.Cu") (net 2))
 (segment (start 98.249 79.749) (end 99.5 81) (width 0.3) (layer "F.Cu") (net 2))
 (segment (start 104.649 85.680999) (end 103.25 87.079999) (width 0.3) (layer "F.Cu") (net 2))
 (segment (start 99.5 81) (end 99.5 83.1875) (width 0.3) (layer "F.Cu") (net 2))
 (segment (start 98.249 77.188006) (end 98.249 79.749) (width 0.3) (layer "F.Cu") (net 2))
 (segment (start 115.226134 75.881) (end 108.31324 75.881) (width 0.3) (layer "F.Cu") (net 2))
 (segment (start 104.649 83.944708) (end 104.649 85.680999) (width 0.3) (layer "F.Cu") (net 2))
 (segment (start 104.043291 83.338999) (end 104.649 83.944708) (width 0.3) (layer "F.Cu") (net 2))
 (segment (start 113.23 77.27) (end 116.81 77.27) (width 0.3) (layer "F.Cu") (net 2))
 (segment (start 107.639 74.530528) (end 103.747471 70.638999) (width 0.3) (layer "F.Cu") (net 2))
 (segment (start 107.639 75.20676) (end 107.639 74.530528) (width 0.3) (layer "F.Cu") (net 2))
 (segment (start 113 77.5) (end 113.23 77.27) (width 0.3) (layer "F.Cu") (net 2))
 (segment (start 101.851 71.606106) (end 100.9 72.557106) (width 0.3) (layer "F.Cu") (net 2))
 (segment (start 108.31324 75.881) (end 107.639 75.20676) (width 0.3) (layer "F.Cu") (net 2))
 (segment (start 124.649 82.73329) (end 124.649 85.101) (width 0.3) (layer "F.Cu") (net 2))
 (segment (start 100.9 74.537006) (end 98.249 77.188006) (width 0.3) (layer "F.Cu") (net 2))
 (via (at 119 86.75) (size 3) (drill 0.9) (layers "F.Cu" "B.Cu") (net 2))
 (via (at 113 77.5) (size 3) (drill 0.9) (layers "F.Cu" "B.Cu") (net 2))
 (via (at 117.287006 83.212994) (size 3) (drill 0.9) (layers "F.Cu" "B.Cu") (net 2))
 (via (at 123 86.75) (size 3) (drill 0.9) (layers "F.Cu" "B.Cu") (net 2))
 (segment (start 119 86.75) (end 123 86.75) (width 0.3) (layer "B.Cu") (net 2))
 (segment (start 113 77.5) (end 113 80.5) (width 0.3) (layer "B.Cu") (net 2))
 (segment (start 113 80.5) (end 115.712994 83.212994) (width 0.3) (layer "B.Cu") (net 2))
 (segment (start 115.712994 83.212994) (end 117.287006 83.212994) (width 0.3) (layer "B.Cu") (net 2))
 (segment (start 147 67) (end 147 68) (width 0.3) (layer "F.Cu") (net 10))
 (segment (start 131.020554 68.75) (end 119.36771 68.75) (width 0.3) (layer "F.Cu") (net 10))
 (segment (start 119.36771 68.75) (end 117.26671 66.649) (width 0.3) (layer "F.Cu") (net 10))
 (segment (start 103.600001 77.27) (end 104.470938 77.27) (width 0.3) (layer "F.Cu") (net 10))
 (segment (start 134.889788 72.619234) (end 131.020554 68.75) (width 0.3) (layer "F.Cu") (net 10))
 (segment (start 147 68) (end 138.85 76.15) (width 0.3) (layer "F.Cu") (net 10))
 (segment (start 108.125267 77.27) (end 109.19 77.27) (width 0.3) (layer "F.Cu") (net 10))
 (segment (start 138.85 76.15) (end 136.212994 76.15) (width 0.3) (layer "F.Cu") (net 10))
 (segment (start 108.125268 77.27) (end 108.49 77.27) (width 0.3) (layer "F.Cu") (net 10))
 (segment (start 117.26671 66.649) (end 113.101 66.649) (width 0.3) (layer "F.Cu") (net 10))
 (segment (start 134.889788 74.826794) (end 134.889788 72.619234) (width 0.3) (layer "F.Cu") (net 10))
 (segment (start 136.212994 76.15) (end 134.889788 74.826794) (width 0.3) (layer "F.Cu") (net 10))
 (segment (start 149 67) (end 147 67) (width 0.3) (layer "F.Cu") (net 10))
 (segment (start 150 68) (end 149 67) (width 0.3) (layer "F.Cu") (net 10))
 (segment (start 106.425306 78.969961) (end 108.125268 77.27) (width 0.3) (layer "F.Cu") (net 10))
 (segment (start 104.470938 77.27) (end 106.170899 78.969961) (width 0.3) (layer "F.Cu") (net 10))
 (segment (start 106.425306 78.969961) (end 108.125267 77.27) (width 0.3) (layer "F.Cu") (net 10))
 (segment (start 106.170899 78.969961) (end 106.425306 78.969961) (width 0.3) (layer "F.Cu") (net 10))
 (segment (start 113.101 66.649) (end 112.5 67.25) (width 0.3) (layer "F.Cu") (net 10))
 (via (at 106.425306 78.969961) (size 3) (drill 0.9) (layers "F.Cu" "B.Cu") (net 10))
 (via (at 112.5 67.25) (size 3) (drill 0.9) (layers "F.Cu" "B.Cu") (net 10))
 (segment (start 112.5 67.25) (end 111.25 68.5) (width 0.3) (layer "B.Cu") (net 10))
 (segment (start 110.06676 75.881) (end 108.619 75.881) (width 0.3) (layer "B.Cu") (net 10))
 (segment (start 111.25 68.5) (end 111.25 74.69776) (width 0.3) (layer "B.Cu") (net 10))
 (segment (start 108.619 75.881) (end 106.425306 78.074694) (width 0.3) (layer "B.Cu") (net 10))
 (segment (start 106.425306 78.074694) (end 106.425306 78.969961) (width 0.3) (layer "B.Cu") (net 10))
 (segment (start 111.25 74.69776) (end 110.06676 75.881) (width 0.3) (layer "B.Cu") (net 10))
 (segment (start 114.01571 66.148) (end 117.47423 66.148) (width 0.3) (layer "F.Cu") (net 23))
 (segment (start 103.25 69.299998) (end 102.049 68.098998) (width 0.3) (layer "F.Cu") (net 23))
 (segment (start 119.47623 68.15) (end 141.057107 68.15) (width 0.3) (layer "F.Cu") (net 23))
 (segment (start 117.47423 66.148) (end 119.47623 68.15) (width 0.3) (layer "F.Cu") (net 23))
 (segment (start 113.26671 65.399) (end 114.01571 66.148) (width 0.3) (layer "F.Cu") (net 23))
 (segment (start 102.049 66.262528) (end 102.912528 65.399) (width 0.3) (layer "F.Cu") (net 23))
 (segment (start 141.057107 68.15) (end 143.207106 66) (width 0.3) (layer "F.Cu") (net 23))
 (segment (start 102.049 68.098998) (end 102.049 66.262528) (width 0.3) (layer "F.Cu") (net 23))
 (segment (start 102.912528 65.399) (end 113.26671 65.399) (width 0.3) (layer "F.Cu") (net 23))
 (segment (start 143.207106 66) (end 144.5 66) (width 0.3) (layer "F.Cu") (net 23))
 (segment (start 104.533094 79) (end 104.533094 79.694045) (width 0.3) (layer "F.Cu") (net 15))
 (segment (start 129.90876 73.579) (end 132.68676 73.579) (width 0.3) (layer "F.Cu") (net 15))
 (segment (start 132.68676 73.579) (end 135.75776 76.65) (width 0.3) (layer "F.Cu") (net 15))
 (segment (start 104.488472 79) (end 104.533094 79) (width 0.3) (layer "F.Cu") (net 15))
 (segment (start 112.476006 80.961) (end 115.016006 78.421) (width 0.3) (layer "F.Cu") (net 15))
 (segment (start 103.25 71.839999) (end 101.75 73.339999) (width 0.3) (layer "F.Cu") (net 15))
 (segment (start 101.75 73.339999) (end 101.75 77.5) (width 0.3) (layer "F.Cu") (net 15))
 (segment (start 125.06676 78.421) (end 129.90876 73.579) (width 0.3) (layer "F.Cu") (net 15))
 (segment (start 102.508999 78.258999) (end 103.747471 78.258999) (width 0.3) (layer "F.Cu") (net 15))
 (segment (start 135.75776 76.65) (end 142.019999 76.65) (width 0.3) (layer "F.Cu") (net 15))
 (segment (start 142.019999 76.65) (end 144.5 74.169999) (width 0.3) (layer "F.Cu") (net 15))
 (segment (start 104.533094 79.694045) (end 105.800049 80.961) (width 0.3) (layer "F.Cu") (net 15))
 (segment (start 115.016006 78.421) (end 125.06676 78.421) (width 0.3) (layer "F.Cu") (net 15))
 (segment (start 105.800049 80.961) (end 112.476006 80.961) (width 0.3) (layer "F.Cu") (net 15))
 (segment (start 101.75 77.5) (end 102.508999 78.258999) (width 0.3) (layer "F.Cu") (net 15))
 (segment (start 103.747471 78.258999) (end 104.488472 79) (width 0.3) (layer "F.Cu") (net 15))
 (segment (start 115.259 70.197885) (end 116.718432 68.738453) (width 0.3) (layer "F.Cu") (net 7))
 (segment (start 111.05 87.9) (end 114.65 87.9) (width 0.3) (layer "F.Cu") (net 7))
 (segment (start 114.65 87.9) (end 116.5 89.75) (width 0.3) (layer "F.Cu") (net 7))
 (segment (start 152 68) (end 152 65) (width 0.3) (layer "F.Cu") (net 7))
 (segment (start 116.5 89.75) (end 149.25 89.75) (width 0.3) (layer "F.Cu") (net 7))
 (segment (start 152 87) (end 152 79) (width 0.3) (layer "F.Cu") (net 7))
 (segment (start 116.81 74.73) (end 115.259 73.179) (width 0.3) (layer "F.Cu") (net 7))
 (segment (start 115.259 73.179) (end 115.259 70.197885) (width 0.3) (layer "F.Cu") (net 7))
 (segment (start 149.25 89.75) (end 152 87) (width 0.3) (layer "F.Cu") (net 7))
 (segment (start 152 71) (end 152 68) (width 0.3) (layer "F.Cu") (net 7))
 (segment (start 152 71) (end 152 79) (width 0.3) (layer "F.Cu") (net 7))
 (segment (start 111 87.85) (end 111.05 87.9) (width 0.3) (layer "F.Cu") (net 7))
 (via (at 111 87.85) (size 3) (drill 0.9) (layers "F.Cu" "B.Cu") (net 7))
 (via (at 116.718432 68.738453) (size 3) (drill 0.9) (layers "F.Cu" "B.Cu") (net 7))
 (segment (start 111 76.812994) (end 115.259 72.553994) (width 0.3) (layer "B.Cu") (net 7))
 (segment (start 115.259 72.553994) (end 115.259 70.197885) (width 0.3) (layer "B.Cu") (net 7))
 (segment (start 111 87.85) (end 111 76.812994) (width 0.3) (layer "B.Cu") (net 7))
 (segment (start 115.259 70.197885) (end 116.718432 68.738453) (width 0.3) (layer "B.Cu") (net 7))
 (segment (start 150 87) (end 147.34 87) (width 0.3) (layer "F.Cu") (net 6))
 (segment (start 139 87) (end 141.66 87) (width 0.3) (layer "F.Cu") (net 4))
 (segment (start 137 79) (end 136.08 79) (width 0.3) (layer "F.Cu") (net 3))
 (segment (start 147 65.141902) (end 144.980902 67.161) (width 0.3) (layer "F.Cu") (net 3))
 (segment (start 133.25 83.75) (end 137 80) (width 0.3) (layer "F.Cu") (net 3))
 (segment (start 137 79) (end 137 87) (width 0.3) (layer "F.Cu") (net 3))
 (segment (start 142.753214 67.161) (end 141.264214 68.65) (width 0.3) (layer "F.Cu") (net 3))
 (segment (start 137 71) (end 137 74.25) (width 0.3) (layer "F.Cu") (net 3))
 (segment (start 137 80) (end 137 79) (width 0.3) (layer "F.Cu") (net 3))
 (segment (start 136.08 79) (end 131.81 74.73) (width 0.3) (layer "F.Cu") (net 3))
 (segment (start 141.264214 68.65) (end 139.35 68.65) (width 0.3) (layer "F.Cu") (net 3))
 (segment (start 135 87) (end 137 87) (width 0.3) (layer "F.Cu") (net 3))
 (segment (start 139.35 68.65) (end 137 71) (width 0.3) (layer "F.Cu") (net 3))
 (segment (start 144.980902 67.161) (end 142.753214 67.161) (width 0.3) (layer "F.Cu") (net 3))
 (via (at 137 74.25) (size 3) (drill 0.9) (layers "F.Cu" "B.Cu") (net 3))
 (via (at 133.25 83.75) (size 3) (drill 0.9) (layers "F.Cu" "B.Cu") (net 3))
 (segment (start 137 74.25) (end 137 80) (width 0.3) (layer "B.Cu") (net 3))
 (segment (start 137 80) (end 133.25 83.75) (width 0.3) (layer "B.Cu") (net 3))
 (segment (start 147 79.169999) (end 149.830001 79.169999) (width 0.3) (layer "F.Cu") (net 13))
 (segment (start 139 79) (end 141.830001 79) (width 0.3) (layer "F.Cu") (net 9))
 (segment (start 150 71) (end 147 71) (width 0.3) (layer "F.Cu") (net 14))
 (segment (start 139 71) (end 142 71) (width 0.3) (layer "F.Cu") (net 5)))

